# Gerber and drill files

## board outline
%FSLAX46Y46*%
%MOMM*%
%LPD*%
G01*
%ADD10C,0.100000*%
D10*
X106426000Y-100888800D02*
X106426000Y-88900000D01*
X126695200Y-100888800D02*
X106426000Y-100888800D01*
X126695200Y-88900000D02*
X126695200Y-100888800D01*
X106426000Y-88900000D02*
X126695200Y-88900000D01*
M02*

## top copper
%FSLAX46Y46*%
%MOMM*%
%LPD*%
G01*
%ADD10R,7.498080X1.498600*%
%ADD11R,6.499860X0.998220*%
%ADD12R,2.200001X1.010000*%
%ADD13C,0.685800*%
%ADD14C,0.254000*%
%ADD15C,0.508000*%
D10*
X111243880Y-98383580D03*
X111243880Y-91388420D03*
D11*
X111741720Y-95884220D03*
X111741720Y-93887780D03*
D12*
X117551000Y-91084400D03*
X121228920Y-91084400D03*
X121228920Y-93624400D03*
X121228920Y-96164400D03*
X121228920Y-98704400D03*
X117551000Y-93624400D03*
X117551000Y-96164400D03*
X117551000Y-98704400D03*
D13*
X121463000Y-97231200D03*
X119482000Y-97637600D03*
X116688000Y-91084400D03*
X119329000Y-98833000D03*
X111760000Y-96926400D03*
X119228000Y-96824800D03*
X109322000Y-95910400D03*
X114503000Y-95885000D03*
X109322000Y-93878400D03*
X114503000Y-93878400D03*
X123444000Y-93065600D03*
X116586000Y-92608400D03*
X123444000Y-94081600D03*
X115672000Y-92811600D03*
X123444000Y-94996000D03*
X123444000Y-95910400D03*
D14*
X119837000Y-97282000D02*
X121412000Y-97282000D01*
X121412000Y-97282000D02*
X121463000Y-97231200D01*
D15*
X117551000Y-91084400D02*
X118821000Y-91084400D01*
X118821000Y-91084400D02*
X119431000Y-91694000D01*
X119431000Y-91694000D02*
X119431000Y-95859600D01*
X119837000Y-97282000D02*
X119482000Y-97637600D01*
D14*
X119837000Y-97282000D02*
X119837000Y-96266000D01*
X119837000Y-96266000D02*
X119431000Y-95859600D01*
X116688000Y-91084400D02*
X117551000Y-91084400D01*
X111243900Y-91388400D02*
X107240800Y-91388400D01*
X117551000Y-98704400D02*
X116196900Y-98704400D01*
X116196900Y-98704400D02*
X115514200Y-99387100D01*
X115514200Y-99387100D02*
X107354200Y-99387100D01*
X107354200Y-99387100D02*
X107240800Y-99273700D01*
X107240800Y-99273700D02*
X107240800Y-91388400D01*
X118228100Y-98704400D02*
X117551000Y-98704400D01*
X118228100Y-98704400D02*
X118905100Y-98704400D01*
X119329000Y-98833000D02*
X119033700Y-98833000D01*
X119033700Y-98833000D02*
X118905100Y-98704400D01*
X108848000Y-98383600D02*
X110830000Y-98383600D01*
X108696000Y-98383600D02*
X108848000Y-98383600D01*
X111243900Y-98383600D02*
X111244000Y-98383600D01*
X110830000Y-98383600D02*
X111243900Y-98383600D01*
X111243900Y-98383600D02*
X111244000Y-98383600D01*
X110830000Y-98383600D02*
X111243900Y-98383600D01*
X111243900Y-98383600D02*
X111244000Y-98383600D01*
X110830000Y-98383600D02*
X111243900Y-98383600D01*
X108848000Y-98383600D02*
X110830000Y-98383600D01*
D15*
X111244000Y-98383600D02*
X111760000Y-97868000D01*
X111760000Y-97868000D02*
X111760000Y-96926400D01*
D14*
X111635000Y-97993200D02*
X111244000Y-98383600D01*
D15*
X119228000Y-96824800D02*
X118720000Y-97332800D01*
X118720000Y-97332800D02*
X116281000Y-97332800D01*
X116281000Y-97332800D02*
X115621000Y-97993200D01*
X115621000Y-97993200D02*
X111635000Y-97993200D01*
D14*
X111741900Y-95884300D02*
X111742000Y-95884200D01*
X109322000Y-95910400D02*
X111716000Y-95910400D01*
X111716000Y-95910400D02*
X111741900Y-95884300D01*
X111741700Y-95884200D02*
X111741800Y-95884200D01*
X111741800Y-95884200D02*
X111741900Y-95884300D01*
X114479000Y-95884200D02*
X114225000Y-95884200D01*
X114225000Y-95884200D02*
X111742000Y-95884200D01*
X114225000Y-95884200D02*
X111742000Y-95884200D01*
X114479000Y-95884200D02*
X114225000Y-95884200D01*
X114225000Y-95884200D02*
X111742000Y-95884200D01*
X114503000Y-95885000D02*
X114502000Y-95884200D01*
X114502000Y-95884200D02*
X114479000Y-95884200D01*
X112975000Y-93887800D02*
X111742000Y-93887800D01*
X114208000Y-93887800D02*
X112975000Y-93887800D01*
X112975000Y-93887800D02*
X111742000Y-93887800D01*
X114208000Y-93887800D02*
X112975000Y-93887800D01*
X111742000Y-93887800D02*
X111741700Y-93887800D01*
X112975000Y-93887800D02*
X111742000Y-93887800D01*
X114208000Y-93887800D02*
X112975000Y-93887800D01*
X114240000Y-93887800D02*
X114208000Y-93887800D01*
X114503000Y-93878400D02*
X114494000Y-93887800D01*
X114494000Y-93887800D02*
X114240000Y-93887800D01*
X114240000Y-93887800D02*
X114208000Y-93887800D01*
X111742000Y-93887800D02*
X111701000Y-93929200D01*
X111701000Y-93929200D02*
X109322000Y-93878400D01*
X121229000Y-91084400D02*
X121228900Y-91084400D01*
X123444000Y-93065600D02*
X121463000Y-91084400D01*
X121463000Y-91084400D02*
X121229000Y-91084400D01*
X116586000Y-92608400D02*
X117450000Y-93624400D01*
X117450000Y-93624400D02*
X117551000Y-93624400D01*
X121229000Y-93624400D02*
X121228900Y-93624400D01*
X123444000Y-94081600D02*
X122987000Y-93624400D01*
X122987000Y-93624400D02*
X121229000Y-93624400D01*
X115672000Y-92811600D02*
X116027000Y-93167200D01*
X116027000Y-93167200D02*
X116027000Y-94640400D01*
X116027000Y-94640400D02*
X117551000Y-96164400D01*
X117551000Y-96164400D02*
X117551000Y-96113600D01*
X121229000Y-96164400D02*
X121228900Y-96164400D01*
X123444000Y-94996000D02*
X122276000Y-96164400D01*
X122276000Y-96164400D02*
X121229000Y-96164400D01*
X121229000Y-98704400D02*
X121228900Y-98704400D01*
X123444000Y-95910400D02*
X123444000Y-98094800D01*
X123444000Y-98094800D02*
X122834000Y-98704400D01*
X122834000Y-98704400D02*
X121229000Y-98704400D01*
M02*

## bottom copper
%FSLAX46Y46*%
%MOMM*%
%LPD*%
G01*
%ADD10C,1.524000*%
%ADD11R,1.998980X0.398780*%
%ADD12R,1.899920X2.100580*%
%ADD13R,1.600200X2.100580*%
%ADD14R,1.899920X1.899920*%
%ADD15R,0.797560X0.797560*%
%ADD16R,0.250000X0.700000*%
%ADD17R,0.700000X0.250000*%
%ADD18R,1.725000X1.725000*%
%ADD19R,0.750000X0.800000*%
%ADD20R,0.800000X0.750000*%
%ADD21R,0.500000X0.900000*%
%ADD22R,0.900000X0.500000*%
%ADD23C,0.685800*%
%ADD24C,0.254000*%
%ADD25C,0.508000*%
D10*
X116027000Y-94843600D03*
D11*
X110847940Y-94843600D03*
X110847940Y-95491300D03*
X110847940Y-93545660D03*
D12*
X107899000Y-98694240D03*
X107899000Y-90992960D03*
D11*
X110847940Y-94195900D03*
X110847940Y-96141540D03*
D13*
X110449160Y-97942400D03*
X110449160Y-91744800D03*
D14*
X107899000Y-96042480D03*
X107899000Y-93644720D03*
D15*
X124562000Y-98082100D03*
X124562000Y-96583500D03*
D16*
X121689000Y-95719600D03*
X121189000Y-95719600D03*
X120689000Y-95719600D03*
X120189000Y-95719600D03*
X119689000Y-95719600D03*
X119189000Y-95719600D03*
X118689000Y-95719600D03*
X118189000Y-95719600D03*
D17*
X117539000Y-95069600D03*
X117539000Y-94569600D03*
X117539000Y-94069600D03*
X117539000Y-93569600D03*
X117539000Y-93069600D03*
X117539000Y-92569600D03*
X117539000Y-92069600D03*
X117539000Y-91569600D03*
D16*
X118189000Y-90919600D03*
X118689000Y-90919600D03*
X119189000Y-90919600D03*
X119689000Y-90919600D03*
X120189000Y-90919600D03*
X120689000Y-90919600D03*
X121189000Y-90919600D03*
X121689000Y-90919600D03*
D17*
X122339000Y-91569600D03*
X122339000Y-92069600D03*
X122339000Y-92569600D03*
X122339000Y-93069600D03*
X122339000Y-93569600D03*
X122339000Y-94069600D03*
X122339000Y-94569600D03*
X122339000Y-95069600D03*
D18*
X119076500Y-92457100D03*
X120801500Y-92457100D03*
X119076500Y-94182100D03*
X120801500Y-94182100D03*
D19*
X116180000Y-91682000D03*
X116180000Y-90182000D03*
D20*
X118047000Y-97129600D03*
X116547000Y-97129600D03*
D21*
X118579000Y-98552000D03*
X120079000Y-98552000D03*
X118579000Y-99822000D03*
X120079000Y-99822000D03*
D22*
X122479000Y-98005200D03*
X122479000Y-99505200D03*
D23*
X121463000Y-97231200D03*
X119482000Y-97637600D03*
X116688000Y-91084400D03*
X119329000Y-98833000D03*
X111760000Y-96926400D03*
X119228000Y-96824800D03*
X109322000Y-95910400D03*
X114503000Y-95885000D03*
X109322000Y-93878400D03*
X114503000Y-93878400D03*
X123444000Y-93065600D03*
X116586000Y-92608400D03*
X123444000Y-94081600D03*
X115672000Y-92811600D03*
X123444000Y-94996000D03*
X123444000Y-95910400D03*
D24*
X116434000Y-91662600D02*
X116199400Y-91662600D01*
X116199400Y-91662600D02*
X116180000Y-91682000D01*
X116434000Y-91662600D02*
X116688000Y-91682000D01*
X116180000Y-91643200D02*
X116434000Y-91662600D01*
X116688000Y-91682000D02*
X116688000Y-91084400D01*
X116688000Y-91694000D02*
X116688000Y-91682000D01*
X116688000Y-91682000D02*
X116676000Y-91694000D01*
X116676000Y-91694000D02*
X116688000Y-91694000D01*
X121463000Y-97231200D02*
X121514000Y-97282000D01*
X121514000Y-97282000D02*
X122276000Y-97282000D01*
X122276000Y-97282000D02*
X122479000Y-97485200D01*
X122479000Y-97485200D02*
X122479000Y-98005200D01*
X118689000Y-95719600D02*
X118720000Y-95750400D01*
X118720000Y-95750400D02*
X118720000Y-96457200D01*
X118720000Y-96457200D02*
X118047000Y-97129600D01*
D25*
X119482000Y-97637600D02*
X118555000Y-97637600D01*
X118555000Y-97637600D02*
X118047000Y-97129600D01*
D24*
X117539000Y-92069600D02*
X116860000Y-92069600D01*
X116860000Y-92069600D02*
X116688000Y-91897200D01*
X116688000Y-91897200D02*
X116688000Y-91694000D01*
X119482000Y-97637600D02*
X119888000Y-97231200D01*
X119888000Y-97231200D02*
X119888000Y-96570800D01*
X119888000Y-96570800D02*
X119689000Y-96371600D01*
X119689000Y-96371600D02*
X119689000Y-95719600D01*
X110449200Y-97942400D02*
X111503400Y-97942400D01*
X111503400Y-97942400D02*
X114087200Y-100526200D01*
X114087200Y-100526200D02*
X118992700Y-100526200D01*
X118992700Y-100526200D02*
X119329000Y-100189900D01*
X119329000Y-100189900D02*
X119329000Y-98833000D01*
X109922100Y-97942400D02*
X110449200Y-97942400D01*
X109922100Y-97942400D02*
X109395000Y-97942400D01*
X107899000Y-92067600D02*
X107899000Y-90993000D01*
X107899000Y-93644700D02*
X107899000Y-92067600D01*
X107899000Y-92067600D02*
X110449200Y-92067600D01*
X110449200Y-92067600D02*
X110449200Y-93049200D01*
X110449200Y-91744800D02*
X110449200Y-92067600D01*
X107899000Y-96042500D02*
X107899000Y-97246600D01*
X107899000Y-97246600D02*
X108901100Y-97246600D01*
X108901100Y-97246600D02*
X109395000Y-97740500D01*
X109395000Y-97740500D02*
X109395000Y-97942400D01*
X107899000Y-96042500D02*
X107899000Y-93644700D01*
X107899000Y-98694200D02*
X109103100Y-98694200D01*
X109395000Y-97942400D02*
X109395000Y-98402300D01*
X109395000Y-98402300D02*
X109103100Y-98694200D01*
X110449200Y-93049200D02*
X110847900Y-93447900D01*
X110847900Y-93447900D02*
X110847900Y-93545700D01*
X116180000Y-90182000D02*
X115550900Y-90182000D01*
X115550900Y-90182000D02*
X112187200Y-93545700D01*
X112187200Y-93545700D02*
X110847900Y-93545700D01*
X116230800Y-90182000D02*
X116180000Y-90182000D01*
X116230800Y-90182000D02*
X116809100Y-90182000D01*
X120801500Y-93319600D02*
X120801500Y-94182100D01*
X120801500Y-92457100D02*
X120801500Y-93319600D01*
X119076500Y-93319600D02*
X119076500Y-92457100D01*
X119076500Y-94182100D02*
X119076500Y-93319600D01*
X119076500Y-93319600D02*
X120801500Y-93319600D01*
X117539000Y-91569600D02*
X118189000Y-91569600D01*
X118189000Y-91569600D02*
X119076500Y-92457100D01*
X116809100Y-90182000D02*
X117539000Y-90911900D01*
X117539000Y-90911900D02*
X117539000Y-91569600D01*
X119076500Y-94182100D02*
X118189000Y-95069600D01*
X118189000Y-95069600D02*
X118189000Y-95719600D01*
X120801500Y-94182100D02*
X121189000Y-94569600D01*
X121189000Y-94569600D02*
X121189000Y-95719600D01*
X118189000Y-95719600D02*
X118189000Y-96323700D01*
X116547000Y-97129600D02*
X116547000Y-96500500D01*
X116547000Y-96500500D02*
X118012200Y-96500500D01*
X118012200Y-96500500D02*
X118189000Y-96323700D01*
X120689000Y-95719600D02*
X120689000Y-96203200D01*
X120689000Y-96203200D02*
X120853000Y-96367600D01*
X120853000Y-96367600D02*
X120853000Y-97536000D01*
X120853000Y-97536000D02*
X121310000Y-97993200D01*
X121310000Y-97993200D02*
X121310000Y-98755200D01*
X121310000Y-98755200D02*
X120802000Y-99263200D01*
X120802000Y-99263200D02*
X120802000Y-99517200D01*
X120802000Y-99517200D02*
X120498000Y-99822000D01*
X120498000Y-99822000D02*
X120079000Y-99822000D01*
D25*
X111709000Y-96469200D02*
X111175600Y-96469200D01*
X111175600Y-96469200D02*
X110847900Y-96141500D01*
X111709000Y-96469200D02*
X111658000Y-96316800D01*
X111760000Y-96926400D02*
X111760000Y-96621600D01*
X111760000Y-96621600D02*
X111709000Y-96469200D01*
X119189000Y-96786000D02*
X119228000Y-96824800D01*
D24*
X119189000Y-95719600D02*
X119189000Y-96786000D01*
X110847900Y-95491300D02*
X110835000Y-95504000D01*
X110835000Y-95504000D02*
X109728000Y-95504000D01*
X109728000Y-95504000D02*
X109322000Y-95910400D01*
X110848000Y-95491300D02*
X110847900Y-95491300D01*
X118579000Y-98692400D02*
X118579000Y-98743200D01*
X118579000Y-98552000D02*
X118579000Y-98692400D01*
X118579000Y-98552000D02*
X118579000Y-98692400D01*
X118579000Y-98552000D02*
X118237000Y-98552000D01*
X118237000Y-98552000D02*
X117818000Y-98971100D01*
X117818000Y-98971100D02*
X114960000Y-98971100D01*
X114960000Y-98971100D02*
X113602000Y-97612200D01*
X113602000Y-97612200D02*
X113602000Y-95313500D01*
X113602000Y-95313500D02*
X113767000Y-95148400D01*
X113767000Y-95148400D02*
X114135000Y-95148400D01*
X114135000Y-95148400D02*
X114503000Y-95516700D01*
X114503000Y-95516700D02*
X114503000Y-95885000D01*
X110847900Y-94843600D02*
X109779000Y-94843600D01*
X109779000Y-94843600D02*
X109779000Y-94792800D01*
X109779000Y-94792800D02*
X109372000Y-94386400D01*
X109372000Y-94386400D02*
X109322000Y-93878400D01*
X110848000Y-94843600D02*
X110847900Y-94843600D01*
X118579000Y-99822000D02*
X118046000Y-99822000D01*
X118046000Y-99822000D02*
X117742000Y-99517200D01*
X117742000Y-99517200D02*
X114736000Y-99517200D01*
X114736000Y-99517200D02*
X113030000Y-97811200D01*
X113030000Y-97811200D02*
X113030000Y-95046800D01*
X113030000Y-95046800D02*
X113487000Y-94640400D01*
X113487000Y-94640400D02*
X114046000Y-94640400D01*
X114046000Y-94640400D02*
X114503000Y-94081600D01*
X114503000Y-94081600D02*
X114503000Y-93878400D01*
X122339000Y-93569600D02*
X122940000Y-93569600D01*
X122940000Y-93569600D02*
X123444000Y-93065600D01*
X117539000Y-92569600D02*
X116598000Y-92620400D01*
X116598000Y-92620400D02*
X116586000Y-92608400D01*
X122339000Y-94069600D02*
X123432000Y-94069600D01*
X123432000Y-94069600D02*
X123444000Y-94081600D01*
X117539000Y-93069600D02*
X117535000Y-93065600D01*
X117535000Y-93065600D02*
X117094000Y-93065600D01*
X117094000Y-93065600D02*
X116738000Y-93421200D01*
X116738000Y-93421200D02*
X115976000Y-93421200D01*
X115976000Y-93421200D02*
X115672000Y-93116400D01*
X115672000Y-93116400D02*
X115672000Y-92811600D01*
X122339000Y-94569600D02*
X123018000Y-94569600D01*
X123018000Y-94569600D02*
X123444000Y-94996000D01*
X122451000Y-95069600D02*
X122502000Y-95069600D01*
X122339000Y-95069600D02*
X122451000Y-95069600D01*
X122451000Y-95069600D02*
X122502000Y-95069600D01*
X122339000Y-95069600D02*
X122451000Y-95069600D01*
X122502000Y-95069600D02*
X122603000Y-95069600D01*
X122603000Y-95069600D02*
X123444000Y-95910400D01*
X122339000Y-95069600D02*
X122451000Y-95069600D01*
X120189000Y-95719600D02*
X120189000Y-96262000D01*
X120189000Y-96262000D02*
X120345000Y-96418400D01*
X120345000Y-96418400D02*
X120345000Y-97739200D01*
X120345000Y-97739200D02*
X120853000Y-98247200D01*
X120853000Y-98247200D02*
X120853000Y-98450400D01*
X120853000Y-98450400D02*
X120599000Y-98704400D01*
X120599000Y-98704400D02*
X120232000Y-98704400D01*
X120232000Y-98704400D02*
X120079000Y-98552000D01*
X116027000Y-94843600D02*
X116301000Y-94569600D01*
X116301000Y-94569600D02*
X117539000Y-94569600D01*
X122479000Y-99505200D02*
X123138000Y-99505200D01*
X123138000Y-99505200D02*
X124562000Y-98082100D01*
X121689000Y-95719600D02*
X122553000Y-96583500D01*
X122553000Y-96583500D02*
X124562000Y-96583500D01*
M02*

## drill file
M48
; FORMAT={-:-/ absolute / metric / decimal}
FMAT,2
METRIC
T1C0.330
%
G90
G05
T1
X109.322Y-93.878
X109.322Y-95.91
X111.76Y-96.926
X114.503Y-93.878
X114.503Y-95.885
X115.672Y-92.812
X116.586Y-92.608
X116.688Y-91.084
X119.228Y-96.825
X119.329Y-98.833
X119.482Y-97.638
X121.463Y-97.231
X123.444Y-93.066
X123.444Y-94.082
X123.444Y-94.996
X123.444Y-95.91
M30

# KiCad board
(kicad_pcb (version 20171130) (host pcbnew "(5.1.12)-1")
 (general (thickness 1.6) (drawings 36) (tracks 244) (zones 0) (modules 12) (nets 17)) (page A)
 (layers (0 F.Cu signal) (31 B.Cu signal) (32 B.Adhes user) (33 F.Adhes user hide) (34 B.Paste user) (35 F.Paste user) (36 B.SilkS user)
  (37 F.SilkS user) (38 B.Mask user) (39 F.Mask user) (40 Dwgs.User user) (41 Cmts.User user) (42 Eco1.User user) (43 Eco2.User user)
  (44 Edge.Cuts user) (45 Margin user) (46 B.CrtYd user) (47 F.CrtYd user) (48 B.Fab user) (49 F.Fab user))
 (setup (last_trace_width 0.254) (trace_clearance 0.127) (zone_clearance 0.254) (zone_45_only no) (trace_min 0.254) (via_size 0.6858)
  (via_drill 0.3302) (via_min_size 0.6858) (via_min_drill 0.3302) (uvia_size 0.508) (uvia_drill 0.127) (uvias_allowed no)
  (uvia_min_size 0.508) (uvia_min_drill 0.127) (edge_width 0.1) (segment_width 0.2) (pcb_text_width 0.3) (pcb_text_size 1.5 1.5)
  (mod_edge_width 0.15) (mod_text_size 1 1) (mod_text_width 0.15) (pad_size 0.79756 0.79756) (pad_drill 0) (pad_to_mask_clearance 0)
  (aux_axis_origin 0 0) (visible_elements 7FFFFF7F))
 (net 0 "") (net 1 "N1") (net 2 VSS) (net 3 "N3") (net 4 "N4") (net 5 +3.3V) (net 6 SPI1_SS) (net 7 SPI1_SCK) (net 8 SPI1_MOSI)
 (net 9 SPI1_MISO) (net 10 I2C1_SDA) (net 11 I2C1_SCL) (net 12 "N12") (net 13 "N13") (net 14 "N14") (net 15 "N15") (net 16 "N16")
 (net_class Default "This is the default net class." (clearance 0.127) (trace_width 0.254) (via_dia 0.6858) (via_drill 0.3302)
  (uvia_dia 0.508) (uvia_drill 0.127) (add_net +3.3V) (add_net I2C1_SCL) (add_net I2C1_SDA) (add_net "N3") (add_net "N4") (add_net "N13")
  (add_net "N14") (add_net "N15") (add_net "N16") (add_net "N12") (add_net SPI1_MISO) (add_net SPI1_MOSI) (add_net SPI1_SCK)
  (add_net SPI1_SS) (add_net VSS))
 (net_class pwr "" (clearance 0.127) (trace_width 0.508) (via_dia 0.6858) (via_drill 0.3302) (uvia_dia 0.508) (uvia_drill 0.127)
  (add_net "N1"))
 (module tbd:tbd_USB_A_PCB (layer F.Cu) (at 111.442 94.886)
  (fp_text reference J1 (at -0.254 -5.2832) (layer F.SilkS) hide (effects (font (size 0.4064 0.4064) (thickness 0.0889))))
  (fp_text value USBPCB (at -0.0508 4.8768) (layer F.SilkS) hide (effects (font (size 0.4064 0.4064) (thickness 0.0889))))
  (pad 5V smd rect (at -0.19812 3.49758) (size 7.49808 1.4986) (layers F.Cu F.Paste F.Mask) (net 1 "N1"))
  (pad GND smd rect (at -0.19812 -3.49758) (size 7.49808 1.4986) (layers F.Cu F.Paste F.Mask) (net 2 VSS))
  (pad DN smd rect (at 0.29972 0.99822) (size 6.49986 0.99822) (layers F.Cu F.Paste F.Mask) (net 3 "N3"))
  (pad DP smd rect (at 0.29972 -0.99822) (size 6.49986 0.99822) (layers F.Cu F.Paste F.Mask) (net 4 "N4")))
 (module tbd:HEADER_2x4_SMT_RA (layer F.Cu) (at 117.551 91.0844 90)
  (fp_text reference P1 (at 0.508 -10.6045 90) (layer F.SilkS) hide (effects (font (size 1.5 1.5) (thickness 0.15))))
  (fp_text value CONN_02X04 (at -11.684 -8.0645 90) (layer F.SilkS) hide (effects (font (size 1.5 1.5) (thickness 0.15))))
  (pad 1 smd rect (at 0 0 90) (size 1.01 2.200001) (layers F.Cu F.Paste F.Mask) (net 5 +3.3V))
  (pad 2 smd rect (at 0 3.67792 90) (size 1.01 2.200001) (layers F.Cu F.Paste F.Mask) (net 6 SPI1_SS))
  (pad 4 smd rect (at -2.54 3.67792 90) (size 1.01 2.200001) (layers F.Cu F.Paste F.Mask) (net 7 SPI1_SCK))
  (pad 6 smd rect (at -5.08 3.67792 90) (size 1.01 2.200001) (layers F.Cu F.Paste F.Mask) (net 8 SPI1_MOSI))
  (pad 8 smd rect (at -7.62 3.67792 90) (size 1.01 2.200001) (layers F.Cu F.Paste F.Mask) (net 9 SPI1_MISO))
  (pad 3 smd rect (at -2.54 0 90) (size 1.01 2.200001) (layers F.Cu F.Paste F.Mask) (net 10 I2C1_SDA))
  (pad 5 smd rect (at -5.08 0 90) (size 1.01 2.200001) (layers F.Cu F.Paste F.Mask) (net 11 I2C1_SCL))
  (pad 7 smd rect (at -7.62 0 90) (size 1.01 2.200001) (layers F.Cu F.Paste F.Mask) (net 2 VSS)))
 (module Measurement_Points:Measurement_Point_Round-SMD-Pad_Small (layer B.Cu) (at 116.027 94.8436)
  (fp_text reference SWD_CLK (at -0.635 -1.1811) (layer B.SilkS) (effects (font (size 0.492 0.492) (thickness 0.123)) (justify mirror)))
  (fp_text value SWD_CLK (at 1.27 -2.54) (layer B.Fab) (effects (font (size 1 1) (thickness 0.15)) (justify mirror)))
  (pad 1 smd circle (at 0 0) (size 1.524 1.524) (layers B.Cu B.Paste B.Mask) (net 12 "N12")))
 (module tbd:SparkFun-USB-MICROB (layer B.Cu) (at 107.899 94.8436 90)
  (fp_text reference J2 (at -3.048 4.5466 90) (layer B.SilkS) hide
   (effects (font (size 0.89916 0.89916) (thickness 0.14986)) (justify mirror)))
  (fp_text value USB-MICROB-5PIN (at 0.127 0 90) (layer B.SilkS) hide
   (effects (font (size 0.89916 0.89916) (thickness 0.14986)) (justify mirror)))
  (pad D+ smd rect (at 0 2.94894 90) (size 0.39878 1.99898) (layers B.Cu B.Paste B.Mask) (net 4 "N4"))
  (pad D- smd rect (at -0.6477 2.94894 90) (size 0.39878 1.99898) (layers B.Cu B.Paste B.Mask) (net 3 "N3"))
  (pad GND smd rect (at 1.29794 2.94894 90) (size 0.39878 1.99898) (layers B.Cu B.Paste B.Mask) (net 2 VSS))
  (pad MTN2 smd rect (at -3.85064 0 90) (size 2.10058 1.89992) (layers B.Cu B.Paste B.Mask) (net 2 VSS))
  (pad MTN4 smd rect (at 3.85064 0 90) (size 2.10058 1.89992) (layers B.Cu B.Paste B.Mask) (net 2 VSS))
  (pad ID smd rect (at 0.6477 2.94894 90) (size 0.39878 1.99898) (layers B.Cu B.Paste B.Mask))
  (pad VBUS smd rect (at -1.29794 2.94894 90) (size 0.39878 1.99898) (layers B.Cu B.Paste B.Mask) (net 1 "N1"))
  (pad MTN1 smd rect (at -3.0988 2.55016 90) (size 2.10058 1.6002) (layers B.Cu B.Paste B.Mask) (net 2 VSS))
  (pad MTN3 smd rect (at 3.0988 2.55016 90) (size 2.10058 1.6002) (layers B.Cu B.Paste B.Mask) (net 2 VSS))
  (pad MTN5 smd rect (at -1.19888 0 90) (size 1.89992 1.89992) (layers B.Cu B.Paste B.Mask) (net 2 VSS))
  (pad MTN6 smd rect (at 1.19888 0 90) (size 1.89992 1.89992) (layers B.Cu B.Paste B.Mask) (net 2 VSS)))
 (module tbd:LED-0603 (layer B.Cu) (at 124.562 97.3328 90)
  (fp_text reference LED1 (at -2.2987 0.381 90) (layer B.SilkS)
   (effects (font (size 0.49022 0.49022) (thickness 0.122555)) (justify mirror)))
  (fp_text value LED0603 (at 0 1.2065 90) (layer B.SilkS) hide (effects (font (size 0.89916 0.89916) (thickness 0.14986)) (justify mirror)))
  (pad A smd rect (at -0.7493 0 90) (size 0.79756 0.79756) (layers B.Cu B.Paste B.Mask) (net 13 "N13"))
  (pad C smd rect (at 0.7493 0 90) (size 0.79756 0.79756) (layers B.Cu B.Paste B.Mask) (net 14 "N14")))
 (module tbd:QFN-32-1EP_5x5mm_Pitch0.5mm (layer B.Cu) (at 119.939 93.3196 90)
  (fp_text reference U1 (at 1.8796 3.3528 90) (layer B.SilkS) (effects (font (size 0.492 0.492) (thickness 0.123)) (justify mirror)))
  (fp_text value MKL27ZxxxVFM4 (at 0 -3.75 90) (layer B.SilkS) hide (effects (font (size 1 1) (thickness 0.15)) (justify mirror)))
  (pad 1 smd rect (at -2.4 1.75 90) (size 0.7 0.25) (layers B.Cu B.Paste B.Mask) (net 14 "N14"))
  (pad 2 smd rect (at -2.4 1.25 90) (size 0.7 0.25) (layers B.Cu B.Paste B.Mask) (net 2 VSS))
  (pad 3 smd rect (at -2.4 0.75 90) (size 0.7 0.25) (layers B.Cu B.Paste B.Mask) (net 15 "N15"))
  (pad 4 smd rect (at -2.4 0.25 90) (size 0.7 0.25) (layers B.Cu B.Paste B.Mask) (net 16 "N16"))
  (pad 5 smd rect (at -2.4 -0.25 90) (size 0.7 0.25) (layers B.Cu B.Paste B.Mask) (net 5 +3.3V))
  (pad 6 smd rect (at -2.4 -0.75 90) (size 0.7 0.25) (layers B.Cu B.Paste B.Mask) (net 1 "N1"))
  (pad 7 smd rect (at -2.4 -1.25 90) (size 0.7 0.25) (layers B.Cu B.Paste B.Mask) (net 5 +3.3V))
  (pad 8 smd rect (at -2.4 -1.75 90) (size 0.7 0.25) (layers B.Cu B.Paste B.Mask) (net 2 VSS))
  (pad 9 smd rect (at -1.75 -2.4) (size 0.7 0.25) (layers B.Cu B.Paste B.Mask))
  (pad 10 smd rect (at -1.25 -2.4) (size 0.7 0.25) (layers B.Cu B.Paste B.Mask) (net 12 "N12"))
  (pad 11 smd rect (at -0.75 -2.4) (size 0.7 0.25) (layers B.Cu B.Paste B.Mask))
  (pad 12 smd rect (at -0.25 -2.4) (size 0.7 0.25) (layers B.Cu B.Paste B.Mask))
  (pad 13 smd rect (at 0.25 -2.4) (size 0.7 0.25) (layers B.Cu B.Paste B.Mask) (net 11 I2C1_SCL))
  (pad 14 smd rect (at 0.75 -2.4) (size 0.7 0.25) (layers B.Cu B.Paste B.Mask) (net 10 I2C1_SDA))
  (pad 15 smd rect (at 1.25 -2.4) (size 0.7 0.25) (layers B.Cu B.Paste B.Mask) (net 5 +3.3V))
  (pad 16 smd rect (at 1.75 -2.4) (size 0.7 0.25) (layers B.Cu B.Paste B.Mask) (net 2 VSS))
  (pad 17 smd rect (at 2.4 -1.75 90) (size 0.7 0.25) (layers B.Cu B.Paste B.Mask))
  (pad 18 smd rect (at 2.4 -1.25 90) (size 0.7 0.25) (layers B.Cu B.Paste B.Mask))
  (pad 19 smd rect (at 2.4 -0.75 90) (size 0.7 0.25) (layers B.Cu B.Paste B.Mask))
  (pad 20 smd rect (at 2.4 -0.25 90) (size 0.7 0.25) (layers B.Cu B.Paste B.Mask))
  (pad 21 smd rect (at 2.4 0.25 90) (size 0.7 0.25) (layers B.Cu B.Paste B.Mask))
  (pad 22 smd rect (at 2.4 0.75 90) (size 0.7 0.25) (layers B.Cu B.Paste B.Mask))
  (pad 23 smd rect (at 2.4 1.25 90) (size 0.7 0.25) (layers B.Cu B.Paste B.Mask))
  (pad 24 smd rect (at 2.4 1.75 90) (size 0.7 0.25) (layers B.Cu B.Paste B.Mask))
  (pad 25 smd rect (at 1.75 2.4) (size 0.7 0.25) (layers B.Cu B.Paste B.Mask))
  (pad 26 smd rect (at 1.25 2.4) (size 0.7 0.25) (layers B.Cu B.Paste B.Mask))
  (pad 27 smd rect (at 0.75 2.4) (size 0.7 0.25) (layers B.Cu B.Paste B.Mask))
  (pad 28 smd rect (at 0.25 2.4) (size 0.7 0.25) (layers B.Cu B.Paste B.Mask))
  (pad 29 smd rect (at -0.25 2.4) (size 0.7 0.25) (layers B.Cu B.Paste B.Mask) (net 6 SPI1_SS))
  (pad 30 smd rect (at -0.75 2.4) (size 0.7 0.25) (layers B.Cu B.Paste B.Mask) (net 7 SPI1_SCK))
  (pad 31 smd rect (at -1.25 2.4) (size 0.7 0.25) (layers B.Cu B.Paste B.Mask) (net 8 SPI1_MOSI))
  (pad 32 smd rect (at -1.75 2.4) (size 0.7 0.25) (layers B.Cu B.Paste B.Mask) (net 9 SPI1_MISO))
  (pad 33 smd rect (at 0.8625 -0.8625 90) (size 1.725 1.725) (layers B.Cu B.Paste B.Mask) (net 2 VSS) (solder_paste_margin_ratio -0.2))
  (pad 33 smd rect (at 0.8625 0.8625 90) (size 1.725 1.725) (layers B.Cu B.Paste B.Mask) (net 2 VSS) (solder_paste_margin_ratio -0.2))
  (pad 33 smd rect (at -0.8625 -0.8625 90) (size 1.725 1.725) (layers B.Cu B.Paste B.Mask) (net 2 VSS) (solder_paste_margin_ratio -0.2))
  (pad 33 smd rect (at -0.8625 0.8625 90) (size 1.725 1.725) (layers B.Cu B.Paste B.Mask) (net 2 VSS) (solder_paste_margin_ratio -0.2)))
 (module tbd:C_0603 (layer B.Cu) (at 116.18 90.932 90)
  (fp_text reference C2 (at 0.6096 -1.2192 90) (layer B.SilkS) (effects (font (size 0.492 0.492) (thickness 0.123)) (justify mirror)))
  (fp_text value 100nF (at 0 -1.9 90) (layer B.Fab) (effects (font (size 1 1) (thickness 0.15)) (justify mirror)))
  (pad 1 smd rect (at -0.75 0 90) (size 0.8 0.75) (layers B.Cu B.Paste B.Mask) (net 5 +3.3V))
  (pad 2 smd rect (at 0.75 0 90) (size 0.8 0.75) (layers B.Cu B.Paste B.Mask) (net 2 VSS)))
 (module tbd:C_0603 (layer B.Cu) (at 117.297 97.1296 180)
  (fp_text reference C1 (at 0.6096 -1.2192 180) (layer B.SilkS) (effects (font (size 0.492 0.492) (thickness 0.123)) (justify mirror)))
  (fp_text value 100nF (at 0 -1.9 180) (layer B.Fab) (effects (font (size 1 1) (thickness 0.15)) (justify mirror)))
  (pad 1 smd rect (at -0.75 0 180) (size 0.8 0.75) (layers B.Cu B.Paste B.Mask) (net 5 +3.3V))
  (pad 2 smd rect (at 0.75 0 180) (size 0.8 0.75) (layers B.Cu B.Paste B.Mask) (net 2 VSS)))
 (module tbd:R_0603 (layer B.Cu) (at 119.329 98.552)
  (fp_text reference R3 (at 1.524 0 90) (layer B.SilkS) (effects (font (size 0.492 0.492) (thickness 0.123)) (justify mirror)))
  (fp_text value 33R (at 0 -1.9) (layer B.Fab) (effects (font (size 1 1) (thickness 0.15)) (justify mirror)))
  (pad 1 smd rect (at -0.75 0) (size 0.5 0.9) (layers B.Cu B.Paste B.Mask) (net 3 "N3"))
  (pad 2 smd rect (at 0.75 0) (size 0.5 0.9) (layers B.Cu B.Paste B.Mask) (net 16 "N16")))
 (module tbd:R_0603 (layer B.Cu) (at 119.329 99.822)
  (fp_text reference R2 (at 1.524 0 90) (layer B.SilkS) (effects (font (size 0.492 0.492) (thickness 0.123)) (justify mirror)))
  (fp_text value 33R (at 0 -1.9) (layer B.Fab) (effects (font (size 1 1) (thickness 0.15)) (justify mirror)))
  (pad 1 smd rect (at -0.75 0) (size 0.5 0.9) (layers B.Cu B.Paste B.Mask) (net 4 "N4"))
  (pad 2 smd rect (at 0.75 0) (size 0.5 0.9) (layers B.Cu B.Paste B.Mask) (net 15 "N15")))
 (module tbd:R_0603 (layer B.Cu) (at 122.479 98.7552 270)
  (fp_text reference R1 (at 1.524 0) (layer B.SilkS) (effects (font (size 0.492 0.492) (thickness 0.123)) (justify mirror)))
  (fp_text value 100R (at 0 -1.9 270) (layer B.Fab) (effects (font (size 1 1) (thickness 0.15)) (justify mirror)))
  (pad 1 smd rect (at -0.75 0 270) (size 0.5 0.9) (layers B.Cu B.Paste B.Mask) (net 5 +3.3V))
  (pad 2 smd rect (at 0.75 0 270) (size 0.5 0.9) (layers B.Cu B.Paste B.Mask) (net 13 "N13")))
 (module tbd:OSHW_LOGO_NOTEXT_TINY (layer B.Cu) (at 113.8428 98.4504 270)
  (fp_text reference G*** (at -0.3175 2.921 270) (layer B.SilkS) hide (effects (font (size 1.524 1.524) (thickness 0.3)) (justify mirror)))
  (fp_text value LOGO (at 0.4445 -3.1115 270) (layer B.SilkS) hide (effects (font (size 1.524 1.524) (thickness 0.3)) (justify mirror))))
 (gr_line (start 106.426 100.8888) (end 106.426 88.9) (angle 90) (layer Edge.Cuts) (width 0.1))
 (gr_line (start 126.6952 100.8888) (end 106.426 100.8888) (angle 90) (layer Edge.Cuts) (width 0.1))
 (gr_line (start 126.6952 88.9) (end 126.6952 100.8888) (angle 90) (layer Edge.Cuts) (width 0.1))
 (gr_line (start 106.426 88.9) (end 126.6952 88.9) (angle 90) (layer Edge.Cuts) (width 0.1))
 (segment (start 116.434 91.6626) (end 116.1994 91.6626) (width 0.254) (layer B.Cu) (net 5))
 (segment (start 116.1994 91.6626) (end 116.18 91.682) (width 0.254) (layer B.Cu) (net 5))
 (segment (start 116.434 91.6626) (end 116.688 91.682) (width 0.254) (layer B.Cu) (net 5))
 (segment (start 116.18 91.6432) (end 116.434 91.6626) (width 0.254) (layer B.Cu) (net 5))
 (segment (start 116.688 91.682) (end 116.688 91.0844) (width 0.254) (layer B.Cu) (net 5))
 (segment (start 116.688 91.694) (end 116.688 91.682) (width 0.254) (layer B.Cu) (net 5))
 (segment (start 116.688 91.682) (end 116.676 91.694) (width 0.254) (layer B.Cu) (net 5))
 (segment (start 116.676 91.694) (end 116.688 91.694) (width 0.254) (layer B.Cu) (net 5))
 (segment (start 119.837 97.282) (end 121.412 97.282) (width 0.254) (layer F.Cu) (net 5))
 (segment (start 121.412 97.282) (end 121.463 97.2312) (width 0.254) (layer F.Cu) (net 5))
 (segment (start 121.463 97.2312) (end 121.514 97.282) (width 0.254) (layer B.Cu) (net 5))
 (segment (start 121.514 97.282) (end 122.276 97.282) (width 0.254) (layer B.Cu) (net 5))
 (segment (start 122.276 97.282) (end 122.479 97.4852) (width 0.254) (layer B.Cu) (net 5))
 (segment (start 122.479 97.4852) (end 122.479 98.0052) (width 0.254) (layer B.Cu) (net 5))
 (segment (start 118.689 95.7196) (end 118.72 95.7504) (width 0.254) (layer B.Cu) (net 5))
 (segment (start 118.72 95.7504) (end 118.72 96.4572) (width 0.254) (layer B.Cu) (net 5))
 (segment (start 118.72 96.4572) (end 118.047 97.1296) (width 0.254) (layer B.Cu) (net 5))
 (segment (start 119.482 97.6376) (end 118.555 97.6376) (width 0.508) (layer B.Cu) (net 5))
 (segment (start 118.555 97.6376) (end 118.047 97.1296) (width 0.508) (layer B.Cu) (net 5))
 (segment (start 117.551 91.0844) (end 118.821 91.0844) (width 0.508) (layer F.Cu) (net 5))
 (segment (start 118.821 91.0844) (end 119.431 91.694) (width 0.508) (layer F.Cu) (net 5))
 (segment (start 119.431 91.694) (end 119.431 95.8596) (width 0.508) (layer F.Cu) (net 5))
 (segment (start 119.837 97.282) (end 119.482 97.6376) (width 0.508) (layer F.Cu) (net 5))
 (segment (start 119.837 97.282) (end 119.837 96.266) (width 0.254) (layer F.Cu) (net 5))
 (segment (start 119.837 96.266) (end 119.431 95.8596) (width 0.254) (layer F.Cu) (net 5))
 (segment (start 117.539 92.0696) (end 116.86 92.0696) (width 0.254) (layer B.Cu) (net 5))
 (segment (start 116.86 92.0696) (end 116.688 91.8972) (width 0.254) (layer B.Cu) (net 5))
 (segment (start 116.688 91.8972) (end 116.688 91.694) (width 0.254) (layer B.Cu) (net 5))
 (segment (start 116.688 91.0844) (end 117.551 91.0844) (width 0.254) (layer F.Cu) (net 5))
 (segment (start 119.482 97.6376) (end 119.888 97.2312) (width 0.254) (layer B.Cu) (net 5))
 (segment (start 119.888 97.2312) (end 119.888 96.5708) (width 0.254) (layer B.Cu) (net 5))
 (segment (start 119.888 96.5708) (end 119.689 96.3716) (width 0.254) (layer B.Cu) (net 5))
 (segment (start 119.689 96.3716) (end 119.689 95.7196) (width 0.254) (layer B.Cu) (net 5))
 (via (at 121.463 97.2312) (size 0.6858) (layers F.Cu B.Cu) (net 5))
 (via (at 119.482 97.6376) (size 0.6858) (layers F.Cu B.Cu) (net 5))
 (via (at 116.688 91.0844) (size 0.6858) (layers F.Cu B.Cu) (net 5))
 (segment (start 111.2439 91.3884) (end 107.2408 91.3884) (width 0.254) (layer F.Cu) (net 2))
 (segment (start 117.551 98.7044) (end 116.1969 98.7044) (width 0.254) (layer F.Cu) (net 2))
 (segment (start 116.1969 98.7044) (end 115.5142 99.3871) (width 0.254) (layer F.Cu) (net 2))
 (segment (start 115.5142 99.3871) (end 107.3542 99.3871) (width 0.254) (layer F.Cu) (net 2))
 (segment (start 107.3542 99.3871) (end 107.2408 99.2737) (width 0.254) (layer F.Cu) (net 2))
 (segment (start 107.2408 99.2737) (end 107.2408 91.3884) (width 0.254) (layer F.Cu) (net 2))
 (segment (start 118.2281 98.7044) (end 117.551 98.7044) (width 0.254) (layer F.Cu) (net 2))
 (segment (start 118.2281 98.7044) (end 118.9051 98.7044) (width 0.254) (layer F.Cu) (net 2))
 (segment (start 110.4492 97.9424) (end 111.5034 97.9424) (width 0.254) (layer B.Cu) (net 2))
 (segment (start 119.329 98.833) (end 119.0337 98.833) (width 0.254) (layer F.Cu) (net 2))
 (segment (start 119.0337 98.833) (end 118.9051 98.7044) (width 0.254) (layer F.Cu) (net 2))
 (segment (start 111.5034 97.9424) (end 114.0872 100.5262) (width 0.254) (layer B.Cu) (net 2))
 (segment (start 114.0872 100.5262) (end 118.9927 100.5262) (width 0.254) (layer B.Cu) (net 2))
 (segment (start 118.9927 100.5262) (end 119.329 100.1899) (width 0.254) (layer B.Cu) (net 2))
 (segment (start 119.329 100.1899) (end 119.329 98.833) (width 0.254) (layer B.Cu) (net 2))
 (segment (start 109.9221 97.9424) (end 110.4492 97.9424) (width 0.254) (layer B.Cu) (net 2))
 (segment (start 109.9221 97.9424) (end 109.395 97.9424) (width 0.254) (layer B.Cu) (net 2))
 (segment (start 107.899 92.0676) (end 107.899 90.993) (width 0.254) (layer B.Cu) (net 2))
 (segment (start 107.899 93.6447) (end 107.899 92.0676) (width 0.254) (layer B.Cu) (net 2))
 (segment (start 107.899 92.0676) (end 110.4492 92.0676) (width 0.254) (layer B.Cu) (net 2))
 (segment (start 110.4492 92.0676) (end 110.4492 93.0492) (width 0.254) (layer B.Cu) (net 2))
 (segment (start 110.4492 91.7448) (end 110.4492 92.0676) (width 0.254) (layer B.Cu) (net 2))
 (segment (start 107.899 96.0425) (end 107.899 97.2466) (width 0.254) (layer B.Cu) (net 2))
 (segment (start 107.899 97.2466) (end 108.9011 97.2466) (width 0.254) (layer B.Cu) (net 2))
 (segment (start 108.9011 97.2466) (end 109.395 97.7405) (width 0.254) (layer B.Cu) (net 2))
 (segment (start 109.395 97.7405) (end 109.395 97.9424) (width 0.254) (layer B.Cu) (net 2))
 (segment (start 107.899 96.0425) (end 107.899 93.6447) (width 0.254) (layer B.Cu) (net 2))
 (segment (start 107.899 98.6942) (end 109.1031 98.6942) (width 0.254) (layer B.Cu) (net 2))
 (segment (start 109.395 97.9424) (end 109.395 98.4023) (width 0.254) (layer B.Cu) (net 2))
 (segment (start 109.395 98.4023) (end 109.1031 98.6942) (width 0.254) (layer B.Cu) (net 2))
 (segment (start 110.4492 93.0492) (end 110.8479 93.4479) (width 0.254) (layer B.Cu) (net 2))
 (segment (start 110.8479 93.4479) (end 110.8479 93.5457) (width 0.254) (layer B.Cu) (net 2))
 (segment (start 116.18 90.182) (end 115.5509 90.182) (width 0.254) (layer B.Cu) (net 2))
 (segment (start 115.5509 90.182) (end 112.1872 93.5457) (width 0.254) (layer B.Cu) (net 2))
 (segment (start 112.1872 93.5457) (end 110.8479 93.5457) (width 0.254) (layer B.Cu) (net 2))
 (segment (start 116.2308 90.182) (end 116.18 90.182) (width 0.254) (layer B.Cu) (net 2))
 (segment (start 116.2308 90.182) (end 116.8091 90.182) (width 0.254) (layer B.Cu) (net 2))
 (segment (start 120.8015 93.3196) (end 120.8015 94.1821) (width 0.254) (layer B.Cu) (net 2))
 (segment (start 120.8015 92.4571) (end 120.8015 93.3196) (width 0.254) (layer B.Cu) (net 2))
 (segment (start 119.0765 93.3196) (end 119.0765 92.4571) (width 0.254) (layer B.Cu) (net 2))
 (segment (start 119.0765 94.1821) (end 119.0765 93.3196) (width 0.254) (layer B.Cu) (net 2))
 (segment (start 119.0765 93.3196) (end 120.8015 93.3196) (width 0.254) (layer B.Cu) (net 2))
 (segment (start 117.539 91.5696) (end 118.189 91.5696) (width 0.254) (layer B.Cu) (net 2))
 (segment (start 118.189 91.5696) (end 119.0765 92.4571) (width 0.254) (layer B.Cu) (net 2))
 (segment (start 116.8091 90.182) (end 117.539 90.9119) (width 0.254) (layer B.Cu) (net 2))
 (segment (start 117.539 90.9119) (end 117.539 91.5696) (width 0.254) (layer B.Cu) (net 2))
 (segment (start 119.0765 94.1821) (end 118.189 95.0696) (width 0.254) (layer B.Cu) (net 2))
 (segment (start 118.189 95.0696) (end 118.189 95.7196) (width 0.254) (layer B.Cu) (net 2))
 (segment (start 120.8015 94.1821) (end 121.189 94.5696) (width 0.254) (layer B.Cu) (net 2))
 (segment (start 121.189 94.5696) (end 121.189 95.7196) (width 0.254) (layer B.Cu) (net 2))
 (segment (start 118.189 95.7196) (end 118.189 96.3237) (width 0.254) (layer B.Cu) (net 2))
 (segment (start 116.547 97.1296) (end 116.547 96.5005) (width 0.254) (layer B.Cu) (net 2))
 (segment (start 116.547 96.5005) (end 118.0122 96.5005) (width 0.254) (layer B.Cu) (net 2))
 (segment (start 118.0122 96.5005) (end 118.189 96.3237) (width 0.254) (layer B.Cu) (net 2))
 (via (at 119.329 98.833) (size 0.6858) (layers F.Cu B.Cu) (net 2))
 (segment (start 120.689 95.7196) (end 120.689 96.2032) (width 0.254) (layer B.Cu) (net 15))
 (segment (start 120.689 96.2032) (end 120.853 96.3676) (width 0.254) (layer B.Cu) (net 15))
 (segment (start 120.853 96.3676) (end 120.853 97.536) (width 0.254) (layer B.Cu) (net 15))
 (segment (start 120.853 97.536) (end 121.31 97.9932) (width 0.254) (layer B.Cu) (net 15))
 (segment (start 121.31 97.9932) (end 121.31 98.7552) (width 0.254) (layer B.Cu) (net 15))
 (segment (start 121.31 98.7552) (end 120.802 99.2632) (width 0.254) (layer B.Cu) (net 15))
 (segment (start 120.802 99.2632) (end 120.802 99.5172) (width 0.254) (layer B.Cu) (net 15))
 (segment (start 120.802 99.5172) (end 120.498 99.822) (width 0.254) (layer B.Cu) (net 15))
 (segment (start 120.498 99.822) (end 120.079 99.822) (width 0.254) (layer B.Cu) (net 15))
 (segment (start 111.709 96.4692) (end 111.1756 96.4692) (width 0.508) (layer B.Cu) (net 1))
 (segment (start 111.1756 96.4692) (end 110.8479 96.1415) (width 0.508) (layer B.Cu) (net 1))
 (segment (start 111.709 96.4692) (end 111.658 96.3168) (width 0.508) (layer B.Cu) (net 1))
 (segment (start 111.76 96.9264) (end 111.76 96.6216) (width 0.508) (layer B.Cu) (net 1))
 (segment (start 111.76 96.6216) (end 111.709 96.4692) (width 0.508) (layer B.Cu) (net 1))
 (segment (start 108.848 98.3836) (end 110.83 98.3836) (width 0.254) (layer F.Cu) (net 1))
 (segment (start 108.696 98.3836) (end 108.848 98.3836) (width 0.254) (layer F.Cu) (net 1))
 (segment (start 111.2439 98.3836) (end 111.244 98.3836) (width 0.254) (layer F.Cu) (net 1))
 (segment (start 110.83 98.3836) (end 111.2439 98.3836) (width 0.254) (layer F.Cu) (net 1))
 (segment (start 111.2439 98.3836) (end 111.244 98.3836) (width 0.254) (layer F.Cu) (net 1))
 (segment (start 110.83 98.3836) (end 111.2439 98.3836) (width 0.254) (layer F.Cu) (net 1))
 (segment (start 111.2439 98.3836) (end 111.244 98.3836) (width 0.254) (layer F.Cu) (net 1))
 (segment (start 110.83 98.3836) (end 111.2439 98.3836) (width 0.254) (layer F.Cu) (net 1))
 (segment (start 108.848 98.3836) (end 110.83 98.3836) (width 0.254) (layer F.Cu) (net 1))
 (segment (start 111.244 98.3836) (end 111.76 97.868) (width 0.508) (layer F.Cu) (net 1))
 (segment (start 111.76 97.868) (end 111.76 96.9264) (width 0.508) (layer F.Cu) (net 1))
 (segment (start 111.635 97.9932) (end 111.244 98.3836) (width 0.254) (layer F.Cu) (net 1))
 (segment (start 119.189 96.786) (end 119.228 96.8248) (width 0.508) (layer B.Cu) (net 1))
 (segment (start 119.228 96.8248) (end 118.72 97.3328) (width 0.508) (layer F.Cu) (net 1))
 (segment (start 118.72 97.3328) (end 116.281 97.3328) (width 0.508) (layer F.Cu) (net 1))
 (segment (start 116.281 97.3328) (end 115.621 97.9932) (width 0.508) (layer F.Cu) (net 1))
 (segment (start 115.621 97.9932) (end 111.635 97.9932) (width 0.508) (layer F.Cu) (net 1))
 (segment (start 119.189 95.7196) (end 119.189 96.786) (width 0.254) (layer B.Cu) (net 1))
 (via (at 111.76 96.9264) (size 0.6858) (layers F.Cu B.Cu) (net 1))
 (via (at 119.228 96.8248) (size 0.6858) (layers F.Cu B.Cu) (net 1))
 (segment (start 111.7419 95.8843) (end 111.742 95.8842) (width 0.254) (layer F.Cu) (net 3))
 (segment (start 109.322 95.9104) (end 111.716 95.9104) (width 0.254) (layer F.Cu) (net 3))
 (segment (start 111.716 95.9104) (end 111.7419 95.8843) (width 0.254) (layer F.Cu) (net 3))
 (segment (start 111.7417 95.8842) (end 111.7418 95.8842) (width 0.254) (layer F.Cu) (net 3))
 (segment (start 111.7418 95.8842) (end 111.7419 95.8843) (width 0.254) (layer F.Cu) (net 3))
 (segment (start 110.8479 95.4913) (end 110.835 95.504) (width 0.254) (layer B.Cu) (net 3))
 (segment (start 110.835 95.504) (end 109.728 95.504) (width 0.254) (layer B.Cu) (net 3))
 (segment (start 109.728 95.504) (end 109.322 95.9104) (width 0.254) (layer B.Cu) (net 3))
 (segment (start 110.848 95.4913) (end 110.8479 95.4913) (width 0.254) (layer B.Cu) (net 3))
 (segment (start 114.479 95.8842) (end 114.225 95.8842) (width 0.254) (layer F.Cu) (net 3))
 (segment (start 114.225 95.8842) (end 111.742 95.8842) (width 0.254) (layer F.Cu) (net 3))
 (segment (start 114.225 95.8842) (end 111.742 95.8842) (width 0.254) (layer F.Cu) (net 3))
 (segment (start 114.479 95.8842) (end 114.225 95.8842) (width 0.254) (layer F.Cu) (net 3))
 (segment (start 118.579 98.6924) (end 118.579 98.7432) (width 0.254) (layer B.Cu) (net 3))
 (segment (start 118.579 98.552) (end 118.579 98.6924) (width 0.254) (layer B.Cu) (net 3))
 (segment (start 118.579 98.552) (end 118.579 98.6924) (width 0.254) (layer B.Cu) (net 3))
 (segment (start 114.225 95.8842) (end 111.742 95.8842) (width 0.254) (layer F.Cu) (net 3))
 (segment (start 118.579 98.552) (end 118.237 98.552) (width 0.254) (layer B.Cu) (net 3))
 (segment (start 118.237 98.552) (end 117.818 98.9711) (width 0.254) (layer B.Cu) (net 3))
 (segment (start 117.818 98.9711) (end 114.96 98.9711) (width 0.254) (layer B.Cu) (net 3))
 (segment (start 114.96 98.9711) (end 113.602 97.6122) (width 0.254) (layer B.Cu) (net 3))
 (segment (start 113.602 97.6122) (end 113.602 95.3135) (width 0.254) (layer B.Cu) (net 3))
 (segment (start 113.602 95.3135) (end 113.767 95.1484) (width 0.254) (layer B.Cu) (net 3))
 (segment (start 113.767 95.1484) (end 114.135 95.1484) (width 0.254) (layer B.Cu) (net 3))
 (segment (start 114.135 95.1484) (end 114.503 95.5167) (width 0.254) (layer B.Cu) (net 3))
 (segment (start 114.503 95.5167) (end 114.503 95.885) (width 0.254) (layer B.Cu) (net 3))
 (segment (start 114.503 95.885) (end 114.502 95.8842) (width 0.254) (layer F.Cu) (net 3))
 (segment (start 114.502 95.8842) (end 114.479 95.8842) (width 0.254) (layer F.Cu) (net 3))
 (via (at 109.322 95.9104) (size 0.6858) (layers F.Cu B.Cu) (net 3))
 (via (at 114.503 95.885) (size 0.6858) (layers F.Cu B.Cu) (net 3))
 (segment (start 112.975 93.8878) (end 111.742 93.8878) (width 0.254) (layer F.Cu) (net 4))
 (segment (start 114.208 93.8878) (end 112.975 93.8878) (width 0.254) (layer F.Cu) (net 4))
 (segment (start 112.975 93.8878) (end 111.742 93.8878) (width 0.254) (layer F.Cu) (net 4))
 (segment (start 114.208 93.8878) (end 112.975 93.8878) (width 0.254) (layer F.Cu) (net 4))
 (segment (start 111.742 93.8878) (end 111.7417 93.8878) (width 0.254) (layer F.Cu) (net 4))
 (segment (start 112.975 93.8878) (end 111.742 93.8878) (width 0.254) (layer F.Cu) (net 4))
 (segment (start 114.208 93.8878) (end 112.975 93.8878) (width 0.254) (layer F.Cu) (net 4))
 (segment (start 110.8479 94.8436) (end 109.779 94.8436) (width 0.254) (layer B.Cu) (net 4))
 (segment (start 109.779 94.8436) (end 109.779 94.7928) (width 0.254) (layer B.Cu) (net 4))
 (segment (start 109.779 94.7928) (end 109.372 94.3864) (width 0.254) (layer B.Cu) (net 4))
 (segment (start 109.372 94.3864) (end 109.322 93.8784) (width 0.254) (layer B.Cu) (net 4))
 (segment (start 110.848 94.8436) (end 110.8479 94.8436) (width 0.254) (layer B.Cu) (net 4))
 (segment (start 114.24 93.8878) (end 114.208 93.8878) (width 0.254) (layer F.Cu) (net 4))
 (segment (start 114.503 93.8784) (end 114.494 93.8878) (width 0.254) (layer F.Cu) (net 4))
 (segment (start 114.494 93.8878) (end 114.24 93.8878) (width 0.254) (layer F.Cu) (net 4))
 (segment (start 114.24 93.8878) (end 114.208 93.8878) (width 0.254) (layer F.Cu) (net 4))
 (segment (start 111.742 93.8878) (end 111.701 93.9292) (width 0.254) (layer F.Cu) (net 4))
 (segment (start 111.701 93.9292) (end 109.322 93.8784) (width 0.254) (layer F.Cu) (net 4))
 (segment (start 118.579 99.822) (end 118.046 99.822) (width 0.254) (layer B.Cu) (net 4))
 (segment (start 118.046 99.822) (end 117.742 99.5172) (width 0.254) (layer B.Cu) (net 4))
 (segment (start 117.742 99.5172) (end 114.736 99.5172) (width 0.254) (layer B.Cu) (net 4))
 (segment (start 114.736 99.5172) (end 113.03 97.8112) (width 0.254) (layer B.Cu) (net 4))
 (segment (start 113.03 97.8112) (end 113.03 95.0468) (width 0.254) (layer B.Cu) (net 4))
 (segment (start 113.03 95.0468) (end 113.487 94.6404) (width 0.254) (layer B.Cu) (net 4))
 (segment (start 113.487 94.6404) (end 114.046 94.6404) (width 0.254) (layer B.Cu) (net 4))
 (segment (start 114.046 94.6404) (end 114.503 94.0816) (width 0.254) (layer B.Cu) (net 4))
 (segment (start 114.503 94.0816) (end 114.503 93.8784) (width 0.254) (layer B.Cu) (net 4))
 (via (at 109.322 93.8784) (size 0.6858) (layers F.Cu B.Cu) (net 4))
 (via (at 114.503 93.8784) (size 0.6858) (layers F.Cu B.Cu) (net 4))
 (segment (start 121.229 91.0844) (end 121.2289 91.0844) (width 0.254) (layer F.Cu) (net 6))
 (segment (start 123.444 93.0656) (end 121.463 91.0844) (width 0.254) (layer F.Cu) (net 6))
 (segment (start 121.463 91.0844) (end 121.229 91.0844) (width 0.254) (layer F.Cu) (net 6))
 (segment (start 122.339 93.5696) (end 122.94 93.5696) (width 0.254) (layer B.Cu) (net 6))
 (segment (start 122.94 93.5696) (end 123.444 93.0656) (width 0.254) (layer B.Cu) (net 6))
 (via (at 123.444 93.0656) (size 0.6858) (layers F.Cu B.Cu) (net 6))
 (segment (start 116.586 92.6084) (end 117.45 93.6244) (width 0.254) (layer F.Cu) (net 10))
 (segment (start 117.45 93.6244) (end 117.551 93.6244) (width 0.254) (layer F.Cu) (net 10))
 (segment (start 117.539 92.5696) (end 116.598 92.6204) (width 0.254) (layer B.Cu) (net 10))
 (segment (start 116.598 92.6204) (end 116.586 92.6084) (width 0.254) (layer B.Cu) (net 10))
 (via (at 116.586 92.6084) (size 0.6858) (layers F.Cu B.Cu) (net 10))
 (segment (start 121.229 93.6244) (end 121.2289 93.6244) (width 0.254) (layer F.Cu) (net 7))
 (segment (start 123.444 94.0816) (end 122.987 93.6244) (width 0.254) (layer F.Cu) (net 7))
 (segment (start 122.987 93.6244) (end 121.229 93.6244) (width 0.254) (layer F.Cu) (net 7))
 (segment (start 122.339 94.0696) (end 123.432 94.0696) (width 0.254) (layer B.Cu) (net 7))
 (segment (start 123.432 94.0696) (end 123.444 94.0816) (width 0.254) (layer B.Cu) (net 7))
 (via (at 123.444 94.0816) (size 0.6858) (layers F.Cu B.Cu) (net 7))
 (segment (start 117.539 93.0696) (end 117.535 93.0656) (width 0.254) (layer B.Cu) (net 11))
 (segment (start 117.535 93.0656) (end 117.094 93.0656) (width 0.254) (layer B.Cu) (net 11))
 (segment (start 117.094 93.0656) (end 116.738 93.4212) (width 0.254) (layer B.Cu) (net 11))
 (segment (start 116.738 93.4212) (end 115.976 93.4212) (width 0.254) (layer B.Cu) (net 11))
 (segment (start 115.976 93.4212) (end 115.672 93.1164) (width 0.254) (layer B.Cu) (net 11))
 (segment (start 115.672 93.1164) (end 115.672 92.8116) (width 0.254) (layer B.Cu) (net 11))
 (segment (start 115.672 92.8116) (end 116.027 93.1672) (width 0.254) (layer F.Cu) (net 11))
 (segment (start 116.027 93.1672) (end 116.027 94.6404) (width 0.254) (layer F.Cu) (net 11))
 (segment (start 116.027 94.6404) (end 117.551 96.1644) (width 0.254) (layer F.Cu) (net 11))
 (segment (start 117.551 96.1644) (end 117.551 96.1136) (width 0.254) (layer F.Cu) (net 11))
 (via (at 115.672 92.8116) (size 0.6858) (layers F.Cu B.Cu) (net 11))
 (segment (start 121.229 96.1644) (end 121.2289 96.1644) (width 0.254) (layer F.Cu) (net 8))
 (segment (start 123.444 94.996) (end 122.276 96.1644) (width 0.254) (layer F.Cu) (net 8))
 (segment (start 122.276 96.1644) (end 121.229 96.1644) (width 0.254) (layer F.Cu) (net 8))
 (segment (start 122.339 94.5696) (end 123.018 94.5696) (width 0.254) (layer B.Cu) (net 8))
 (segment (start 123.018 94.5696) (end 123.444 94.996) (width 0.254) (layer B.Cu) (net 8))
 (via (at 123.444 94.996) (size 0.6858) (layers F.Cu B.Cu) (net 8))
 (segment (start 121.229 98.7044) (end 121.2289 98.7044) (width 0.254) (layer F.Cu) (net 9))
 (segment (start 123.444 95.9104) (end 123.444 98.0948) (width 0.254) (layer F.Cu) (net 9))
 (segment (start 123.444 98.0948) (end 122.834 98.7044) (width 0.254) (layer F.Cu) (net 9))
 (segment (start 122.834 98.7044) (end 121.229 98.7044) (width 0.254) (layer F.Cu) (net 9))
 (segment (start 122.451 95.0696) (end 122.502 95.0696) (width 0.254) (layer B.Cu) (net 9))
 (segment (start 122.339 95.0696) (end 122.451 95.0696) (width 0.254) (layer B.Cu) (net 9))
 (segment (start 122.451 95.0696) (end 122.502 95.0696) (width 0.254) (layer B.Cu) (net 9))
 (segment (start 122.339 95.0696) (end 122.451 95.0696) (width 0.254) (layer B.Cu) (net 9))
 (segment (start 122.502 95.0696) (end 122.603 95.0696) (width 0.254) (layer B.Cu) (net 9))
 (segment (start 122.603 95.0696) (end 123.444 95.9104) (width 0.254) (layer B.Cu) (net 9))
 (segment (start 122.339 95.0696) (end 122.451 95.0696) (width 0.254) (layer B.Cu) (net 9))
 (via (at 123.444 95.9104) (size 0.6858) (layers F.Cu B.Cu) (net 9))
 (segment (start 120.189 95.7196) (end 120.189 96.262) (width 0.254) (layer B.Cu) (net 16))
 (segment (start 120.189 96.262) (end 120.345 96.4184) (width 0.254) (layer B.Cu) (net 16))
 (segment (start 120.345 96.4184) (end 120.345 97.7392) (width 0.254) (layer B.Cu) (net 16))
 (segment (start 120.345 97.7392) (end 120.853 98.2472) (width 0.254) (layer B.Cu) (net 16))
 (segment (start 120.853 98.2472) (end 120.853 98.4504) (width 0.254) (layer B.Cu) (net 16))
 (segment (start 120.853 98.4504) (end 120.599 98.7044) (width 0.254) (layer B.Cu) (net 16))
 (segment (start 120.599 98.7044) (end 120.232 98.7044) (width 0.254) (layer B.Cu) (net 16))
 (segment (start 120.232 98.7044) (end 120.079 98.552) (width 0.254) (layer B.Cu) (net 16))
 (segment (start 116.027 94.8436) (end 116.301 94.5696) (width 0.254) (layer B.Cu) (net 12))
 (segment (start 116.301 94.5696) (end 117.539 94.5696) (width 0.254) (layer B.Cu) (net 12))
 (segment (start 122.479 99.5052) (end 123.138 99.5052) (width 0.254) (layer B.Cu) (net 13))
 (segment (start 123.138 99.5052) (end 124.562 98.0821) (width 0.254) (layer B.Cu) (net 13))
 (segment (start 121.689 95.7196) (end 122.553 96.5835) (width 0.254) (layer B.Cu) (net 14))
 (segment (start 122.553 96.5835) (end 124.562 96.5835) (width 0.254) (layer B.Cu) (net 14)))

